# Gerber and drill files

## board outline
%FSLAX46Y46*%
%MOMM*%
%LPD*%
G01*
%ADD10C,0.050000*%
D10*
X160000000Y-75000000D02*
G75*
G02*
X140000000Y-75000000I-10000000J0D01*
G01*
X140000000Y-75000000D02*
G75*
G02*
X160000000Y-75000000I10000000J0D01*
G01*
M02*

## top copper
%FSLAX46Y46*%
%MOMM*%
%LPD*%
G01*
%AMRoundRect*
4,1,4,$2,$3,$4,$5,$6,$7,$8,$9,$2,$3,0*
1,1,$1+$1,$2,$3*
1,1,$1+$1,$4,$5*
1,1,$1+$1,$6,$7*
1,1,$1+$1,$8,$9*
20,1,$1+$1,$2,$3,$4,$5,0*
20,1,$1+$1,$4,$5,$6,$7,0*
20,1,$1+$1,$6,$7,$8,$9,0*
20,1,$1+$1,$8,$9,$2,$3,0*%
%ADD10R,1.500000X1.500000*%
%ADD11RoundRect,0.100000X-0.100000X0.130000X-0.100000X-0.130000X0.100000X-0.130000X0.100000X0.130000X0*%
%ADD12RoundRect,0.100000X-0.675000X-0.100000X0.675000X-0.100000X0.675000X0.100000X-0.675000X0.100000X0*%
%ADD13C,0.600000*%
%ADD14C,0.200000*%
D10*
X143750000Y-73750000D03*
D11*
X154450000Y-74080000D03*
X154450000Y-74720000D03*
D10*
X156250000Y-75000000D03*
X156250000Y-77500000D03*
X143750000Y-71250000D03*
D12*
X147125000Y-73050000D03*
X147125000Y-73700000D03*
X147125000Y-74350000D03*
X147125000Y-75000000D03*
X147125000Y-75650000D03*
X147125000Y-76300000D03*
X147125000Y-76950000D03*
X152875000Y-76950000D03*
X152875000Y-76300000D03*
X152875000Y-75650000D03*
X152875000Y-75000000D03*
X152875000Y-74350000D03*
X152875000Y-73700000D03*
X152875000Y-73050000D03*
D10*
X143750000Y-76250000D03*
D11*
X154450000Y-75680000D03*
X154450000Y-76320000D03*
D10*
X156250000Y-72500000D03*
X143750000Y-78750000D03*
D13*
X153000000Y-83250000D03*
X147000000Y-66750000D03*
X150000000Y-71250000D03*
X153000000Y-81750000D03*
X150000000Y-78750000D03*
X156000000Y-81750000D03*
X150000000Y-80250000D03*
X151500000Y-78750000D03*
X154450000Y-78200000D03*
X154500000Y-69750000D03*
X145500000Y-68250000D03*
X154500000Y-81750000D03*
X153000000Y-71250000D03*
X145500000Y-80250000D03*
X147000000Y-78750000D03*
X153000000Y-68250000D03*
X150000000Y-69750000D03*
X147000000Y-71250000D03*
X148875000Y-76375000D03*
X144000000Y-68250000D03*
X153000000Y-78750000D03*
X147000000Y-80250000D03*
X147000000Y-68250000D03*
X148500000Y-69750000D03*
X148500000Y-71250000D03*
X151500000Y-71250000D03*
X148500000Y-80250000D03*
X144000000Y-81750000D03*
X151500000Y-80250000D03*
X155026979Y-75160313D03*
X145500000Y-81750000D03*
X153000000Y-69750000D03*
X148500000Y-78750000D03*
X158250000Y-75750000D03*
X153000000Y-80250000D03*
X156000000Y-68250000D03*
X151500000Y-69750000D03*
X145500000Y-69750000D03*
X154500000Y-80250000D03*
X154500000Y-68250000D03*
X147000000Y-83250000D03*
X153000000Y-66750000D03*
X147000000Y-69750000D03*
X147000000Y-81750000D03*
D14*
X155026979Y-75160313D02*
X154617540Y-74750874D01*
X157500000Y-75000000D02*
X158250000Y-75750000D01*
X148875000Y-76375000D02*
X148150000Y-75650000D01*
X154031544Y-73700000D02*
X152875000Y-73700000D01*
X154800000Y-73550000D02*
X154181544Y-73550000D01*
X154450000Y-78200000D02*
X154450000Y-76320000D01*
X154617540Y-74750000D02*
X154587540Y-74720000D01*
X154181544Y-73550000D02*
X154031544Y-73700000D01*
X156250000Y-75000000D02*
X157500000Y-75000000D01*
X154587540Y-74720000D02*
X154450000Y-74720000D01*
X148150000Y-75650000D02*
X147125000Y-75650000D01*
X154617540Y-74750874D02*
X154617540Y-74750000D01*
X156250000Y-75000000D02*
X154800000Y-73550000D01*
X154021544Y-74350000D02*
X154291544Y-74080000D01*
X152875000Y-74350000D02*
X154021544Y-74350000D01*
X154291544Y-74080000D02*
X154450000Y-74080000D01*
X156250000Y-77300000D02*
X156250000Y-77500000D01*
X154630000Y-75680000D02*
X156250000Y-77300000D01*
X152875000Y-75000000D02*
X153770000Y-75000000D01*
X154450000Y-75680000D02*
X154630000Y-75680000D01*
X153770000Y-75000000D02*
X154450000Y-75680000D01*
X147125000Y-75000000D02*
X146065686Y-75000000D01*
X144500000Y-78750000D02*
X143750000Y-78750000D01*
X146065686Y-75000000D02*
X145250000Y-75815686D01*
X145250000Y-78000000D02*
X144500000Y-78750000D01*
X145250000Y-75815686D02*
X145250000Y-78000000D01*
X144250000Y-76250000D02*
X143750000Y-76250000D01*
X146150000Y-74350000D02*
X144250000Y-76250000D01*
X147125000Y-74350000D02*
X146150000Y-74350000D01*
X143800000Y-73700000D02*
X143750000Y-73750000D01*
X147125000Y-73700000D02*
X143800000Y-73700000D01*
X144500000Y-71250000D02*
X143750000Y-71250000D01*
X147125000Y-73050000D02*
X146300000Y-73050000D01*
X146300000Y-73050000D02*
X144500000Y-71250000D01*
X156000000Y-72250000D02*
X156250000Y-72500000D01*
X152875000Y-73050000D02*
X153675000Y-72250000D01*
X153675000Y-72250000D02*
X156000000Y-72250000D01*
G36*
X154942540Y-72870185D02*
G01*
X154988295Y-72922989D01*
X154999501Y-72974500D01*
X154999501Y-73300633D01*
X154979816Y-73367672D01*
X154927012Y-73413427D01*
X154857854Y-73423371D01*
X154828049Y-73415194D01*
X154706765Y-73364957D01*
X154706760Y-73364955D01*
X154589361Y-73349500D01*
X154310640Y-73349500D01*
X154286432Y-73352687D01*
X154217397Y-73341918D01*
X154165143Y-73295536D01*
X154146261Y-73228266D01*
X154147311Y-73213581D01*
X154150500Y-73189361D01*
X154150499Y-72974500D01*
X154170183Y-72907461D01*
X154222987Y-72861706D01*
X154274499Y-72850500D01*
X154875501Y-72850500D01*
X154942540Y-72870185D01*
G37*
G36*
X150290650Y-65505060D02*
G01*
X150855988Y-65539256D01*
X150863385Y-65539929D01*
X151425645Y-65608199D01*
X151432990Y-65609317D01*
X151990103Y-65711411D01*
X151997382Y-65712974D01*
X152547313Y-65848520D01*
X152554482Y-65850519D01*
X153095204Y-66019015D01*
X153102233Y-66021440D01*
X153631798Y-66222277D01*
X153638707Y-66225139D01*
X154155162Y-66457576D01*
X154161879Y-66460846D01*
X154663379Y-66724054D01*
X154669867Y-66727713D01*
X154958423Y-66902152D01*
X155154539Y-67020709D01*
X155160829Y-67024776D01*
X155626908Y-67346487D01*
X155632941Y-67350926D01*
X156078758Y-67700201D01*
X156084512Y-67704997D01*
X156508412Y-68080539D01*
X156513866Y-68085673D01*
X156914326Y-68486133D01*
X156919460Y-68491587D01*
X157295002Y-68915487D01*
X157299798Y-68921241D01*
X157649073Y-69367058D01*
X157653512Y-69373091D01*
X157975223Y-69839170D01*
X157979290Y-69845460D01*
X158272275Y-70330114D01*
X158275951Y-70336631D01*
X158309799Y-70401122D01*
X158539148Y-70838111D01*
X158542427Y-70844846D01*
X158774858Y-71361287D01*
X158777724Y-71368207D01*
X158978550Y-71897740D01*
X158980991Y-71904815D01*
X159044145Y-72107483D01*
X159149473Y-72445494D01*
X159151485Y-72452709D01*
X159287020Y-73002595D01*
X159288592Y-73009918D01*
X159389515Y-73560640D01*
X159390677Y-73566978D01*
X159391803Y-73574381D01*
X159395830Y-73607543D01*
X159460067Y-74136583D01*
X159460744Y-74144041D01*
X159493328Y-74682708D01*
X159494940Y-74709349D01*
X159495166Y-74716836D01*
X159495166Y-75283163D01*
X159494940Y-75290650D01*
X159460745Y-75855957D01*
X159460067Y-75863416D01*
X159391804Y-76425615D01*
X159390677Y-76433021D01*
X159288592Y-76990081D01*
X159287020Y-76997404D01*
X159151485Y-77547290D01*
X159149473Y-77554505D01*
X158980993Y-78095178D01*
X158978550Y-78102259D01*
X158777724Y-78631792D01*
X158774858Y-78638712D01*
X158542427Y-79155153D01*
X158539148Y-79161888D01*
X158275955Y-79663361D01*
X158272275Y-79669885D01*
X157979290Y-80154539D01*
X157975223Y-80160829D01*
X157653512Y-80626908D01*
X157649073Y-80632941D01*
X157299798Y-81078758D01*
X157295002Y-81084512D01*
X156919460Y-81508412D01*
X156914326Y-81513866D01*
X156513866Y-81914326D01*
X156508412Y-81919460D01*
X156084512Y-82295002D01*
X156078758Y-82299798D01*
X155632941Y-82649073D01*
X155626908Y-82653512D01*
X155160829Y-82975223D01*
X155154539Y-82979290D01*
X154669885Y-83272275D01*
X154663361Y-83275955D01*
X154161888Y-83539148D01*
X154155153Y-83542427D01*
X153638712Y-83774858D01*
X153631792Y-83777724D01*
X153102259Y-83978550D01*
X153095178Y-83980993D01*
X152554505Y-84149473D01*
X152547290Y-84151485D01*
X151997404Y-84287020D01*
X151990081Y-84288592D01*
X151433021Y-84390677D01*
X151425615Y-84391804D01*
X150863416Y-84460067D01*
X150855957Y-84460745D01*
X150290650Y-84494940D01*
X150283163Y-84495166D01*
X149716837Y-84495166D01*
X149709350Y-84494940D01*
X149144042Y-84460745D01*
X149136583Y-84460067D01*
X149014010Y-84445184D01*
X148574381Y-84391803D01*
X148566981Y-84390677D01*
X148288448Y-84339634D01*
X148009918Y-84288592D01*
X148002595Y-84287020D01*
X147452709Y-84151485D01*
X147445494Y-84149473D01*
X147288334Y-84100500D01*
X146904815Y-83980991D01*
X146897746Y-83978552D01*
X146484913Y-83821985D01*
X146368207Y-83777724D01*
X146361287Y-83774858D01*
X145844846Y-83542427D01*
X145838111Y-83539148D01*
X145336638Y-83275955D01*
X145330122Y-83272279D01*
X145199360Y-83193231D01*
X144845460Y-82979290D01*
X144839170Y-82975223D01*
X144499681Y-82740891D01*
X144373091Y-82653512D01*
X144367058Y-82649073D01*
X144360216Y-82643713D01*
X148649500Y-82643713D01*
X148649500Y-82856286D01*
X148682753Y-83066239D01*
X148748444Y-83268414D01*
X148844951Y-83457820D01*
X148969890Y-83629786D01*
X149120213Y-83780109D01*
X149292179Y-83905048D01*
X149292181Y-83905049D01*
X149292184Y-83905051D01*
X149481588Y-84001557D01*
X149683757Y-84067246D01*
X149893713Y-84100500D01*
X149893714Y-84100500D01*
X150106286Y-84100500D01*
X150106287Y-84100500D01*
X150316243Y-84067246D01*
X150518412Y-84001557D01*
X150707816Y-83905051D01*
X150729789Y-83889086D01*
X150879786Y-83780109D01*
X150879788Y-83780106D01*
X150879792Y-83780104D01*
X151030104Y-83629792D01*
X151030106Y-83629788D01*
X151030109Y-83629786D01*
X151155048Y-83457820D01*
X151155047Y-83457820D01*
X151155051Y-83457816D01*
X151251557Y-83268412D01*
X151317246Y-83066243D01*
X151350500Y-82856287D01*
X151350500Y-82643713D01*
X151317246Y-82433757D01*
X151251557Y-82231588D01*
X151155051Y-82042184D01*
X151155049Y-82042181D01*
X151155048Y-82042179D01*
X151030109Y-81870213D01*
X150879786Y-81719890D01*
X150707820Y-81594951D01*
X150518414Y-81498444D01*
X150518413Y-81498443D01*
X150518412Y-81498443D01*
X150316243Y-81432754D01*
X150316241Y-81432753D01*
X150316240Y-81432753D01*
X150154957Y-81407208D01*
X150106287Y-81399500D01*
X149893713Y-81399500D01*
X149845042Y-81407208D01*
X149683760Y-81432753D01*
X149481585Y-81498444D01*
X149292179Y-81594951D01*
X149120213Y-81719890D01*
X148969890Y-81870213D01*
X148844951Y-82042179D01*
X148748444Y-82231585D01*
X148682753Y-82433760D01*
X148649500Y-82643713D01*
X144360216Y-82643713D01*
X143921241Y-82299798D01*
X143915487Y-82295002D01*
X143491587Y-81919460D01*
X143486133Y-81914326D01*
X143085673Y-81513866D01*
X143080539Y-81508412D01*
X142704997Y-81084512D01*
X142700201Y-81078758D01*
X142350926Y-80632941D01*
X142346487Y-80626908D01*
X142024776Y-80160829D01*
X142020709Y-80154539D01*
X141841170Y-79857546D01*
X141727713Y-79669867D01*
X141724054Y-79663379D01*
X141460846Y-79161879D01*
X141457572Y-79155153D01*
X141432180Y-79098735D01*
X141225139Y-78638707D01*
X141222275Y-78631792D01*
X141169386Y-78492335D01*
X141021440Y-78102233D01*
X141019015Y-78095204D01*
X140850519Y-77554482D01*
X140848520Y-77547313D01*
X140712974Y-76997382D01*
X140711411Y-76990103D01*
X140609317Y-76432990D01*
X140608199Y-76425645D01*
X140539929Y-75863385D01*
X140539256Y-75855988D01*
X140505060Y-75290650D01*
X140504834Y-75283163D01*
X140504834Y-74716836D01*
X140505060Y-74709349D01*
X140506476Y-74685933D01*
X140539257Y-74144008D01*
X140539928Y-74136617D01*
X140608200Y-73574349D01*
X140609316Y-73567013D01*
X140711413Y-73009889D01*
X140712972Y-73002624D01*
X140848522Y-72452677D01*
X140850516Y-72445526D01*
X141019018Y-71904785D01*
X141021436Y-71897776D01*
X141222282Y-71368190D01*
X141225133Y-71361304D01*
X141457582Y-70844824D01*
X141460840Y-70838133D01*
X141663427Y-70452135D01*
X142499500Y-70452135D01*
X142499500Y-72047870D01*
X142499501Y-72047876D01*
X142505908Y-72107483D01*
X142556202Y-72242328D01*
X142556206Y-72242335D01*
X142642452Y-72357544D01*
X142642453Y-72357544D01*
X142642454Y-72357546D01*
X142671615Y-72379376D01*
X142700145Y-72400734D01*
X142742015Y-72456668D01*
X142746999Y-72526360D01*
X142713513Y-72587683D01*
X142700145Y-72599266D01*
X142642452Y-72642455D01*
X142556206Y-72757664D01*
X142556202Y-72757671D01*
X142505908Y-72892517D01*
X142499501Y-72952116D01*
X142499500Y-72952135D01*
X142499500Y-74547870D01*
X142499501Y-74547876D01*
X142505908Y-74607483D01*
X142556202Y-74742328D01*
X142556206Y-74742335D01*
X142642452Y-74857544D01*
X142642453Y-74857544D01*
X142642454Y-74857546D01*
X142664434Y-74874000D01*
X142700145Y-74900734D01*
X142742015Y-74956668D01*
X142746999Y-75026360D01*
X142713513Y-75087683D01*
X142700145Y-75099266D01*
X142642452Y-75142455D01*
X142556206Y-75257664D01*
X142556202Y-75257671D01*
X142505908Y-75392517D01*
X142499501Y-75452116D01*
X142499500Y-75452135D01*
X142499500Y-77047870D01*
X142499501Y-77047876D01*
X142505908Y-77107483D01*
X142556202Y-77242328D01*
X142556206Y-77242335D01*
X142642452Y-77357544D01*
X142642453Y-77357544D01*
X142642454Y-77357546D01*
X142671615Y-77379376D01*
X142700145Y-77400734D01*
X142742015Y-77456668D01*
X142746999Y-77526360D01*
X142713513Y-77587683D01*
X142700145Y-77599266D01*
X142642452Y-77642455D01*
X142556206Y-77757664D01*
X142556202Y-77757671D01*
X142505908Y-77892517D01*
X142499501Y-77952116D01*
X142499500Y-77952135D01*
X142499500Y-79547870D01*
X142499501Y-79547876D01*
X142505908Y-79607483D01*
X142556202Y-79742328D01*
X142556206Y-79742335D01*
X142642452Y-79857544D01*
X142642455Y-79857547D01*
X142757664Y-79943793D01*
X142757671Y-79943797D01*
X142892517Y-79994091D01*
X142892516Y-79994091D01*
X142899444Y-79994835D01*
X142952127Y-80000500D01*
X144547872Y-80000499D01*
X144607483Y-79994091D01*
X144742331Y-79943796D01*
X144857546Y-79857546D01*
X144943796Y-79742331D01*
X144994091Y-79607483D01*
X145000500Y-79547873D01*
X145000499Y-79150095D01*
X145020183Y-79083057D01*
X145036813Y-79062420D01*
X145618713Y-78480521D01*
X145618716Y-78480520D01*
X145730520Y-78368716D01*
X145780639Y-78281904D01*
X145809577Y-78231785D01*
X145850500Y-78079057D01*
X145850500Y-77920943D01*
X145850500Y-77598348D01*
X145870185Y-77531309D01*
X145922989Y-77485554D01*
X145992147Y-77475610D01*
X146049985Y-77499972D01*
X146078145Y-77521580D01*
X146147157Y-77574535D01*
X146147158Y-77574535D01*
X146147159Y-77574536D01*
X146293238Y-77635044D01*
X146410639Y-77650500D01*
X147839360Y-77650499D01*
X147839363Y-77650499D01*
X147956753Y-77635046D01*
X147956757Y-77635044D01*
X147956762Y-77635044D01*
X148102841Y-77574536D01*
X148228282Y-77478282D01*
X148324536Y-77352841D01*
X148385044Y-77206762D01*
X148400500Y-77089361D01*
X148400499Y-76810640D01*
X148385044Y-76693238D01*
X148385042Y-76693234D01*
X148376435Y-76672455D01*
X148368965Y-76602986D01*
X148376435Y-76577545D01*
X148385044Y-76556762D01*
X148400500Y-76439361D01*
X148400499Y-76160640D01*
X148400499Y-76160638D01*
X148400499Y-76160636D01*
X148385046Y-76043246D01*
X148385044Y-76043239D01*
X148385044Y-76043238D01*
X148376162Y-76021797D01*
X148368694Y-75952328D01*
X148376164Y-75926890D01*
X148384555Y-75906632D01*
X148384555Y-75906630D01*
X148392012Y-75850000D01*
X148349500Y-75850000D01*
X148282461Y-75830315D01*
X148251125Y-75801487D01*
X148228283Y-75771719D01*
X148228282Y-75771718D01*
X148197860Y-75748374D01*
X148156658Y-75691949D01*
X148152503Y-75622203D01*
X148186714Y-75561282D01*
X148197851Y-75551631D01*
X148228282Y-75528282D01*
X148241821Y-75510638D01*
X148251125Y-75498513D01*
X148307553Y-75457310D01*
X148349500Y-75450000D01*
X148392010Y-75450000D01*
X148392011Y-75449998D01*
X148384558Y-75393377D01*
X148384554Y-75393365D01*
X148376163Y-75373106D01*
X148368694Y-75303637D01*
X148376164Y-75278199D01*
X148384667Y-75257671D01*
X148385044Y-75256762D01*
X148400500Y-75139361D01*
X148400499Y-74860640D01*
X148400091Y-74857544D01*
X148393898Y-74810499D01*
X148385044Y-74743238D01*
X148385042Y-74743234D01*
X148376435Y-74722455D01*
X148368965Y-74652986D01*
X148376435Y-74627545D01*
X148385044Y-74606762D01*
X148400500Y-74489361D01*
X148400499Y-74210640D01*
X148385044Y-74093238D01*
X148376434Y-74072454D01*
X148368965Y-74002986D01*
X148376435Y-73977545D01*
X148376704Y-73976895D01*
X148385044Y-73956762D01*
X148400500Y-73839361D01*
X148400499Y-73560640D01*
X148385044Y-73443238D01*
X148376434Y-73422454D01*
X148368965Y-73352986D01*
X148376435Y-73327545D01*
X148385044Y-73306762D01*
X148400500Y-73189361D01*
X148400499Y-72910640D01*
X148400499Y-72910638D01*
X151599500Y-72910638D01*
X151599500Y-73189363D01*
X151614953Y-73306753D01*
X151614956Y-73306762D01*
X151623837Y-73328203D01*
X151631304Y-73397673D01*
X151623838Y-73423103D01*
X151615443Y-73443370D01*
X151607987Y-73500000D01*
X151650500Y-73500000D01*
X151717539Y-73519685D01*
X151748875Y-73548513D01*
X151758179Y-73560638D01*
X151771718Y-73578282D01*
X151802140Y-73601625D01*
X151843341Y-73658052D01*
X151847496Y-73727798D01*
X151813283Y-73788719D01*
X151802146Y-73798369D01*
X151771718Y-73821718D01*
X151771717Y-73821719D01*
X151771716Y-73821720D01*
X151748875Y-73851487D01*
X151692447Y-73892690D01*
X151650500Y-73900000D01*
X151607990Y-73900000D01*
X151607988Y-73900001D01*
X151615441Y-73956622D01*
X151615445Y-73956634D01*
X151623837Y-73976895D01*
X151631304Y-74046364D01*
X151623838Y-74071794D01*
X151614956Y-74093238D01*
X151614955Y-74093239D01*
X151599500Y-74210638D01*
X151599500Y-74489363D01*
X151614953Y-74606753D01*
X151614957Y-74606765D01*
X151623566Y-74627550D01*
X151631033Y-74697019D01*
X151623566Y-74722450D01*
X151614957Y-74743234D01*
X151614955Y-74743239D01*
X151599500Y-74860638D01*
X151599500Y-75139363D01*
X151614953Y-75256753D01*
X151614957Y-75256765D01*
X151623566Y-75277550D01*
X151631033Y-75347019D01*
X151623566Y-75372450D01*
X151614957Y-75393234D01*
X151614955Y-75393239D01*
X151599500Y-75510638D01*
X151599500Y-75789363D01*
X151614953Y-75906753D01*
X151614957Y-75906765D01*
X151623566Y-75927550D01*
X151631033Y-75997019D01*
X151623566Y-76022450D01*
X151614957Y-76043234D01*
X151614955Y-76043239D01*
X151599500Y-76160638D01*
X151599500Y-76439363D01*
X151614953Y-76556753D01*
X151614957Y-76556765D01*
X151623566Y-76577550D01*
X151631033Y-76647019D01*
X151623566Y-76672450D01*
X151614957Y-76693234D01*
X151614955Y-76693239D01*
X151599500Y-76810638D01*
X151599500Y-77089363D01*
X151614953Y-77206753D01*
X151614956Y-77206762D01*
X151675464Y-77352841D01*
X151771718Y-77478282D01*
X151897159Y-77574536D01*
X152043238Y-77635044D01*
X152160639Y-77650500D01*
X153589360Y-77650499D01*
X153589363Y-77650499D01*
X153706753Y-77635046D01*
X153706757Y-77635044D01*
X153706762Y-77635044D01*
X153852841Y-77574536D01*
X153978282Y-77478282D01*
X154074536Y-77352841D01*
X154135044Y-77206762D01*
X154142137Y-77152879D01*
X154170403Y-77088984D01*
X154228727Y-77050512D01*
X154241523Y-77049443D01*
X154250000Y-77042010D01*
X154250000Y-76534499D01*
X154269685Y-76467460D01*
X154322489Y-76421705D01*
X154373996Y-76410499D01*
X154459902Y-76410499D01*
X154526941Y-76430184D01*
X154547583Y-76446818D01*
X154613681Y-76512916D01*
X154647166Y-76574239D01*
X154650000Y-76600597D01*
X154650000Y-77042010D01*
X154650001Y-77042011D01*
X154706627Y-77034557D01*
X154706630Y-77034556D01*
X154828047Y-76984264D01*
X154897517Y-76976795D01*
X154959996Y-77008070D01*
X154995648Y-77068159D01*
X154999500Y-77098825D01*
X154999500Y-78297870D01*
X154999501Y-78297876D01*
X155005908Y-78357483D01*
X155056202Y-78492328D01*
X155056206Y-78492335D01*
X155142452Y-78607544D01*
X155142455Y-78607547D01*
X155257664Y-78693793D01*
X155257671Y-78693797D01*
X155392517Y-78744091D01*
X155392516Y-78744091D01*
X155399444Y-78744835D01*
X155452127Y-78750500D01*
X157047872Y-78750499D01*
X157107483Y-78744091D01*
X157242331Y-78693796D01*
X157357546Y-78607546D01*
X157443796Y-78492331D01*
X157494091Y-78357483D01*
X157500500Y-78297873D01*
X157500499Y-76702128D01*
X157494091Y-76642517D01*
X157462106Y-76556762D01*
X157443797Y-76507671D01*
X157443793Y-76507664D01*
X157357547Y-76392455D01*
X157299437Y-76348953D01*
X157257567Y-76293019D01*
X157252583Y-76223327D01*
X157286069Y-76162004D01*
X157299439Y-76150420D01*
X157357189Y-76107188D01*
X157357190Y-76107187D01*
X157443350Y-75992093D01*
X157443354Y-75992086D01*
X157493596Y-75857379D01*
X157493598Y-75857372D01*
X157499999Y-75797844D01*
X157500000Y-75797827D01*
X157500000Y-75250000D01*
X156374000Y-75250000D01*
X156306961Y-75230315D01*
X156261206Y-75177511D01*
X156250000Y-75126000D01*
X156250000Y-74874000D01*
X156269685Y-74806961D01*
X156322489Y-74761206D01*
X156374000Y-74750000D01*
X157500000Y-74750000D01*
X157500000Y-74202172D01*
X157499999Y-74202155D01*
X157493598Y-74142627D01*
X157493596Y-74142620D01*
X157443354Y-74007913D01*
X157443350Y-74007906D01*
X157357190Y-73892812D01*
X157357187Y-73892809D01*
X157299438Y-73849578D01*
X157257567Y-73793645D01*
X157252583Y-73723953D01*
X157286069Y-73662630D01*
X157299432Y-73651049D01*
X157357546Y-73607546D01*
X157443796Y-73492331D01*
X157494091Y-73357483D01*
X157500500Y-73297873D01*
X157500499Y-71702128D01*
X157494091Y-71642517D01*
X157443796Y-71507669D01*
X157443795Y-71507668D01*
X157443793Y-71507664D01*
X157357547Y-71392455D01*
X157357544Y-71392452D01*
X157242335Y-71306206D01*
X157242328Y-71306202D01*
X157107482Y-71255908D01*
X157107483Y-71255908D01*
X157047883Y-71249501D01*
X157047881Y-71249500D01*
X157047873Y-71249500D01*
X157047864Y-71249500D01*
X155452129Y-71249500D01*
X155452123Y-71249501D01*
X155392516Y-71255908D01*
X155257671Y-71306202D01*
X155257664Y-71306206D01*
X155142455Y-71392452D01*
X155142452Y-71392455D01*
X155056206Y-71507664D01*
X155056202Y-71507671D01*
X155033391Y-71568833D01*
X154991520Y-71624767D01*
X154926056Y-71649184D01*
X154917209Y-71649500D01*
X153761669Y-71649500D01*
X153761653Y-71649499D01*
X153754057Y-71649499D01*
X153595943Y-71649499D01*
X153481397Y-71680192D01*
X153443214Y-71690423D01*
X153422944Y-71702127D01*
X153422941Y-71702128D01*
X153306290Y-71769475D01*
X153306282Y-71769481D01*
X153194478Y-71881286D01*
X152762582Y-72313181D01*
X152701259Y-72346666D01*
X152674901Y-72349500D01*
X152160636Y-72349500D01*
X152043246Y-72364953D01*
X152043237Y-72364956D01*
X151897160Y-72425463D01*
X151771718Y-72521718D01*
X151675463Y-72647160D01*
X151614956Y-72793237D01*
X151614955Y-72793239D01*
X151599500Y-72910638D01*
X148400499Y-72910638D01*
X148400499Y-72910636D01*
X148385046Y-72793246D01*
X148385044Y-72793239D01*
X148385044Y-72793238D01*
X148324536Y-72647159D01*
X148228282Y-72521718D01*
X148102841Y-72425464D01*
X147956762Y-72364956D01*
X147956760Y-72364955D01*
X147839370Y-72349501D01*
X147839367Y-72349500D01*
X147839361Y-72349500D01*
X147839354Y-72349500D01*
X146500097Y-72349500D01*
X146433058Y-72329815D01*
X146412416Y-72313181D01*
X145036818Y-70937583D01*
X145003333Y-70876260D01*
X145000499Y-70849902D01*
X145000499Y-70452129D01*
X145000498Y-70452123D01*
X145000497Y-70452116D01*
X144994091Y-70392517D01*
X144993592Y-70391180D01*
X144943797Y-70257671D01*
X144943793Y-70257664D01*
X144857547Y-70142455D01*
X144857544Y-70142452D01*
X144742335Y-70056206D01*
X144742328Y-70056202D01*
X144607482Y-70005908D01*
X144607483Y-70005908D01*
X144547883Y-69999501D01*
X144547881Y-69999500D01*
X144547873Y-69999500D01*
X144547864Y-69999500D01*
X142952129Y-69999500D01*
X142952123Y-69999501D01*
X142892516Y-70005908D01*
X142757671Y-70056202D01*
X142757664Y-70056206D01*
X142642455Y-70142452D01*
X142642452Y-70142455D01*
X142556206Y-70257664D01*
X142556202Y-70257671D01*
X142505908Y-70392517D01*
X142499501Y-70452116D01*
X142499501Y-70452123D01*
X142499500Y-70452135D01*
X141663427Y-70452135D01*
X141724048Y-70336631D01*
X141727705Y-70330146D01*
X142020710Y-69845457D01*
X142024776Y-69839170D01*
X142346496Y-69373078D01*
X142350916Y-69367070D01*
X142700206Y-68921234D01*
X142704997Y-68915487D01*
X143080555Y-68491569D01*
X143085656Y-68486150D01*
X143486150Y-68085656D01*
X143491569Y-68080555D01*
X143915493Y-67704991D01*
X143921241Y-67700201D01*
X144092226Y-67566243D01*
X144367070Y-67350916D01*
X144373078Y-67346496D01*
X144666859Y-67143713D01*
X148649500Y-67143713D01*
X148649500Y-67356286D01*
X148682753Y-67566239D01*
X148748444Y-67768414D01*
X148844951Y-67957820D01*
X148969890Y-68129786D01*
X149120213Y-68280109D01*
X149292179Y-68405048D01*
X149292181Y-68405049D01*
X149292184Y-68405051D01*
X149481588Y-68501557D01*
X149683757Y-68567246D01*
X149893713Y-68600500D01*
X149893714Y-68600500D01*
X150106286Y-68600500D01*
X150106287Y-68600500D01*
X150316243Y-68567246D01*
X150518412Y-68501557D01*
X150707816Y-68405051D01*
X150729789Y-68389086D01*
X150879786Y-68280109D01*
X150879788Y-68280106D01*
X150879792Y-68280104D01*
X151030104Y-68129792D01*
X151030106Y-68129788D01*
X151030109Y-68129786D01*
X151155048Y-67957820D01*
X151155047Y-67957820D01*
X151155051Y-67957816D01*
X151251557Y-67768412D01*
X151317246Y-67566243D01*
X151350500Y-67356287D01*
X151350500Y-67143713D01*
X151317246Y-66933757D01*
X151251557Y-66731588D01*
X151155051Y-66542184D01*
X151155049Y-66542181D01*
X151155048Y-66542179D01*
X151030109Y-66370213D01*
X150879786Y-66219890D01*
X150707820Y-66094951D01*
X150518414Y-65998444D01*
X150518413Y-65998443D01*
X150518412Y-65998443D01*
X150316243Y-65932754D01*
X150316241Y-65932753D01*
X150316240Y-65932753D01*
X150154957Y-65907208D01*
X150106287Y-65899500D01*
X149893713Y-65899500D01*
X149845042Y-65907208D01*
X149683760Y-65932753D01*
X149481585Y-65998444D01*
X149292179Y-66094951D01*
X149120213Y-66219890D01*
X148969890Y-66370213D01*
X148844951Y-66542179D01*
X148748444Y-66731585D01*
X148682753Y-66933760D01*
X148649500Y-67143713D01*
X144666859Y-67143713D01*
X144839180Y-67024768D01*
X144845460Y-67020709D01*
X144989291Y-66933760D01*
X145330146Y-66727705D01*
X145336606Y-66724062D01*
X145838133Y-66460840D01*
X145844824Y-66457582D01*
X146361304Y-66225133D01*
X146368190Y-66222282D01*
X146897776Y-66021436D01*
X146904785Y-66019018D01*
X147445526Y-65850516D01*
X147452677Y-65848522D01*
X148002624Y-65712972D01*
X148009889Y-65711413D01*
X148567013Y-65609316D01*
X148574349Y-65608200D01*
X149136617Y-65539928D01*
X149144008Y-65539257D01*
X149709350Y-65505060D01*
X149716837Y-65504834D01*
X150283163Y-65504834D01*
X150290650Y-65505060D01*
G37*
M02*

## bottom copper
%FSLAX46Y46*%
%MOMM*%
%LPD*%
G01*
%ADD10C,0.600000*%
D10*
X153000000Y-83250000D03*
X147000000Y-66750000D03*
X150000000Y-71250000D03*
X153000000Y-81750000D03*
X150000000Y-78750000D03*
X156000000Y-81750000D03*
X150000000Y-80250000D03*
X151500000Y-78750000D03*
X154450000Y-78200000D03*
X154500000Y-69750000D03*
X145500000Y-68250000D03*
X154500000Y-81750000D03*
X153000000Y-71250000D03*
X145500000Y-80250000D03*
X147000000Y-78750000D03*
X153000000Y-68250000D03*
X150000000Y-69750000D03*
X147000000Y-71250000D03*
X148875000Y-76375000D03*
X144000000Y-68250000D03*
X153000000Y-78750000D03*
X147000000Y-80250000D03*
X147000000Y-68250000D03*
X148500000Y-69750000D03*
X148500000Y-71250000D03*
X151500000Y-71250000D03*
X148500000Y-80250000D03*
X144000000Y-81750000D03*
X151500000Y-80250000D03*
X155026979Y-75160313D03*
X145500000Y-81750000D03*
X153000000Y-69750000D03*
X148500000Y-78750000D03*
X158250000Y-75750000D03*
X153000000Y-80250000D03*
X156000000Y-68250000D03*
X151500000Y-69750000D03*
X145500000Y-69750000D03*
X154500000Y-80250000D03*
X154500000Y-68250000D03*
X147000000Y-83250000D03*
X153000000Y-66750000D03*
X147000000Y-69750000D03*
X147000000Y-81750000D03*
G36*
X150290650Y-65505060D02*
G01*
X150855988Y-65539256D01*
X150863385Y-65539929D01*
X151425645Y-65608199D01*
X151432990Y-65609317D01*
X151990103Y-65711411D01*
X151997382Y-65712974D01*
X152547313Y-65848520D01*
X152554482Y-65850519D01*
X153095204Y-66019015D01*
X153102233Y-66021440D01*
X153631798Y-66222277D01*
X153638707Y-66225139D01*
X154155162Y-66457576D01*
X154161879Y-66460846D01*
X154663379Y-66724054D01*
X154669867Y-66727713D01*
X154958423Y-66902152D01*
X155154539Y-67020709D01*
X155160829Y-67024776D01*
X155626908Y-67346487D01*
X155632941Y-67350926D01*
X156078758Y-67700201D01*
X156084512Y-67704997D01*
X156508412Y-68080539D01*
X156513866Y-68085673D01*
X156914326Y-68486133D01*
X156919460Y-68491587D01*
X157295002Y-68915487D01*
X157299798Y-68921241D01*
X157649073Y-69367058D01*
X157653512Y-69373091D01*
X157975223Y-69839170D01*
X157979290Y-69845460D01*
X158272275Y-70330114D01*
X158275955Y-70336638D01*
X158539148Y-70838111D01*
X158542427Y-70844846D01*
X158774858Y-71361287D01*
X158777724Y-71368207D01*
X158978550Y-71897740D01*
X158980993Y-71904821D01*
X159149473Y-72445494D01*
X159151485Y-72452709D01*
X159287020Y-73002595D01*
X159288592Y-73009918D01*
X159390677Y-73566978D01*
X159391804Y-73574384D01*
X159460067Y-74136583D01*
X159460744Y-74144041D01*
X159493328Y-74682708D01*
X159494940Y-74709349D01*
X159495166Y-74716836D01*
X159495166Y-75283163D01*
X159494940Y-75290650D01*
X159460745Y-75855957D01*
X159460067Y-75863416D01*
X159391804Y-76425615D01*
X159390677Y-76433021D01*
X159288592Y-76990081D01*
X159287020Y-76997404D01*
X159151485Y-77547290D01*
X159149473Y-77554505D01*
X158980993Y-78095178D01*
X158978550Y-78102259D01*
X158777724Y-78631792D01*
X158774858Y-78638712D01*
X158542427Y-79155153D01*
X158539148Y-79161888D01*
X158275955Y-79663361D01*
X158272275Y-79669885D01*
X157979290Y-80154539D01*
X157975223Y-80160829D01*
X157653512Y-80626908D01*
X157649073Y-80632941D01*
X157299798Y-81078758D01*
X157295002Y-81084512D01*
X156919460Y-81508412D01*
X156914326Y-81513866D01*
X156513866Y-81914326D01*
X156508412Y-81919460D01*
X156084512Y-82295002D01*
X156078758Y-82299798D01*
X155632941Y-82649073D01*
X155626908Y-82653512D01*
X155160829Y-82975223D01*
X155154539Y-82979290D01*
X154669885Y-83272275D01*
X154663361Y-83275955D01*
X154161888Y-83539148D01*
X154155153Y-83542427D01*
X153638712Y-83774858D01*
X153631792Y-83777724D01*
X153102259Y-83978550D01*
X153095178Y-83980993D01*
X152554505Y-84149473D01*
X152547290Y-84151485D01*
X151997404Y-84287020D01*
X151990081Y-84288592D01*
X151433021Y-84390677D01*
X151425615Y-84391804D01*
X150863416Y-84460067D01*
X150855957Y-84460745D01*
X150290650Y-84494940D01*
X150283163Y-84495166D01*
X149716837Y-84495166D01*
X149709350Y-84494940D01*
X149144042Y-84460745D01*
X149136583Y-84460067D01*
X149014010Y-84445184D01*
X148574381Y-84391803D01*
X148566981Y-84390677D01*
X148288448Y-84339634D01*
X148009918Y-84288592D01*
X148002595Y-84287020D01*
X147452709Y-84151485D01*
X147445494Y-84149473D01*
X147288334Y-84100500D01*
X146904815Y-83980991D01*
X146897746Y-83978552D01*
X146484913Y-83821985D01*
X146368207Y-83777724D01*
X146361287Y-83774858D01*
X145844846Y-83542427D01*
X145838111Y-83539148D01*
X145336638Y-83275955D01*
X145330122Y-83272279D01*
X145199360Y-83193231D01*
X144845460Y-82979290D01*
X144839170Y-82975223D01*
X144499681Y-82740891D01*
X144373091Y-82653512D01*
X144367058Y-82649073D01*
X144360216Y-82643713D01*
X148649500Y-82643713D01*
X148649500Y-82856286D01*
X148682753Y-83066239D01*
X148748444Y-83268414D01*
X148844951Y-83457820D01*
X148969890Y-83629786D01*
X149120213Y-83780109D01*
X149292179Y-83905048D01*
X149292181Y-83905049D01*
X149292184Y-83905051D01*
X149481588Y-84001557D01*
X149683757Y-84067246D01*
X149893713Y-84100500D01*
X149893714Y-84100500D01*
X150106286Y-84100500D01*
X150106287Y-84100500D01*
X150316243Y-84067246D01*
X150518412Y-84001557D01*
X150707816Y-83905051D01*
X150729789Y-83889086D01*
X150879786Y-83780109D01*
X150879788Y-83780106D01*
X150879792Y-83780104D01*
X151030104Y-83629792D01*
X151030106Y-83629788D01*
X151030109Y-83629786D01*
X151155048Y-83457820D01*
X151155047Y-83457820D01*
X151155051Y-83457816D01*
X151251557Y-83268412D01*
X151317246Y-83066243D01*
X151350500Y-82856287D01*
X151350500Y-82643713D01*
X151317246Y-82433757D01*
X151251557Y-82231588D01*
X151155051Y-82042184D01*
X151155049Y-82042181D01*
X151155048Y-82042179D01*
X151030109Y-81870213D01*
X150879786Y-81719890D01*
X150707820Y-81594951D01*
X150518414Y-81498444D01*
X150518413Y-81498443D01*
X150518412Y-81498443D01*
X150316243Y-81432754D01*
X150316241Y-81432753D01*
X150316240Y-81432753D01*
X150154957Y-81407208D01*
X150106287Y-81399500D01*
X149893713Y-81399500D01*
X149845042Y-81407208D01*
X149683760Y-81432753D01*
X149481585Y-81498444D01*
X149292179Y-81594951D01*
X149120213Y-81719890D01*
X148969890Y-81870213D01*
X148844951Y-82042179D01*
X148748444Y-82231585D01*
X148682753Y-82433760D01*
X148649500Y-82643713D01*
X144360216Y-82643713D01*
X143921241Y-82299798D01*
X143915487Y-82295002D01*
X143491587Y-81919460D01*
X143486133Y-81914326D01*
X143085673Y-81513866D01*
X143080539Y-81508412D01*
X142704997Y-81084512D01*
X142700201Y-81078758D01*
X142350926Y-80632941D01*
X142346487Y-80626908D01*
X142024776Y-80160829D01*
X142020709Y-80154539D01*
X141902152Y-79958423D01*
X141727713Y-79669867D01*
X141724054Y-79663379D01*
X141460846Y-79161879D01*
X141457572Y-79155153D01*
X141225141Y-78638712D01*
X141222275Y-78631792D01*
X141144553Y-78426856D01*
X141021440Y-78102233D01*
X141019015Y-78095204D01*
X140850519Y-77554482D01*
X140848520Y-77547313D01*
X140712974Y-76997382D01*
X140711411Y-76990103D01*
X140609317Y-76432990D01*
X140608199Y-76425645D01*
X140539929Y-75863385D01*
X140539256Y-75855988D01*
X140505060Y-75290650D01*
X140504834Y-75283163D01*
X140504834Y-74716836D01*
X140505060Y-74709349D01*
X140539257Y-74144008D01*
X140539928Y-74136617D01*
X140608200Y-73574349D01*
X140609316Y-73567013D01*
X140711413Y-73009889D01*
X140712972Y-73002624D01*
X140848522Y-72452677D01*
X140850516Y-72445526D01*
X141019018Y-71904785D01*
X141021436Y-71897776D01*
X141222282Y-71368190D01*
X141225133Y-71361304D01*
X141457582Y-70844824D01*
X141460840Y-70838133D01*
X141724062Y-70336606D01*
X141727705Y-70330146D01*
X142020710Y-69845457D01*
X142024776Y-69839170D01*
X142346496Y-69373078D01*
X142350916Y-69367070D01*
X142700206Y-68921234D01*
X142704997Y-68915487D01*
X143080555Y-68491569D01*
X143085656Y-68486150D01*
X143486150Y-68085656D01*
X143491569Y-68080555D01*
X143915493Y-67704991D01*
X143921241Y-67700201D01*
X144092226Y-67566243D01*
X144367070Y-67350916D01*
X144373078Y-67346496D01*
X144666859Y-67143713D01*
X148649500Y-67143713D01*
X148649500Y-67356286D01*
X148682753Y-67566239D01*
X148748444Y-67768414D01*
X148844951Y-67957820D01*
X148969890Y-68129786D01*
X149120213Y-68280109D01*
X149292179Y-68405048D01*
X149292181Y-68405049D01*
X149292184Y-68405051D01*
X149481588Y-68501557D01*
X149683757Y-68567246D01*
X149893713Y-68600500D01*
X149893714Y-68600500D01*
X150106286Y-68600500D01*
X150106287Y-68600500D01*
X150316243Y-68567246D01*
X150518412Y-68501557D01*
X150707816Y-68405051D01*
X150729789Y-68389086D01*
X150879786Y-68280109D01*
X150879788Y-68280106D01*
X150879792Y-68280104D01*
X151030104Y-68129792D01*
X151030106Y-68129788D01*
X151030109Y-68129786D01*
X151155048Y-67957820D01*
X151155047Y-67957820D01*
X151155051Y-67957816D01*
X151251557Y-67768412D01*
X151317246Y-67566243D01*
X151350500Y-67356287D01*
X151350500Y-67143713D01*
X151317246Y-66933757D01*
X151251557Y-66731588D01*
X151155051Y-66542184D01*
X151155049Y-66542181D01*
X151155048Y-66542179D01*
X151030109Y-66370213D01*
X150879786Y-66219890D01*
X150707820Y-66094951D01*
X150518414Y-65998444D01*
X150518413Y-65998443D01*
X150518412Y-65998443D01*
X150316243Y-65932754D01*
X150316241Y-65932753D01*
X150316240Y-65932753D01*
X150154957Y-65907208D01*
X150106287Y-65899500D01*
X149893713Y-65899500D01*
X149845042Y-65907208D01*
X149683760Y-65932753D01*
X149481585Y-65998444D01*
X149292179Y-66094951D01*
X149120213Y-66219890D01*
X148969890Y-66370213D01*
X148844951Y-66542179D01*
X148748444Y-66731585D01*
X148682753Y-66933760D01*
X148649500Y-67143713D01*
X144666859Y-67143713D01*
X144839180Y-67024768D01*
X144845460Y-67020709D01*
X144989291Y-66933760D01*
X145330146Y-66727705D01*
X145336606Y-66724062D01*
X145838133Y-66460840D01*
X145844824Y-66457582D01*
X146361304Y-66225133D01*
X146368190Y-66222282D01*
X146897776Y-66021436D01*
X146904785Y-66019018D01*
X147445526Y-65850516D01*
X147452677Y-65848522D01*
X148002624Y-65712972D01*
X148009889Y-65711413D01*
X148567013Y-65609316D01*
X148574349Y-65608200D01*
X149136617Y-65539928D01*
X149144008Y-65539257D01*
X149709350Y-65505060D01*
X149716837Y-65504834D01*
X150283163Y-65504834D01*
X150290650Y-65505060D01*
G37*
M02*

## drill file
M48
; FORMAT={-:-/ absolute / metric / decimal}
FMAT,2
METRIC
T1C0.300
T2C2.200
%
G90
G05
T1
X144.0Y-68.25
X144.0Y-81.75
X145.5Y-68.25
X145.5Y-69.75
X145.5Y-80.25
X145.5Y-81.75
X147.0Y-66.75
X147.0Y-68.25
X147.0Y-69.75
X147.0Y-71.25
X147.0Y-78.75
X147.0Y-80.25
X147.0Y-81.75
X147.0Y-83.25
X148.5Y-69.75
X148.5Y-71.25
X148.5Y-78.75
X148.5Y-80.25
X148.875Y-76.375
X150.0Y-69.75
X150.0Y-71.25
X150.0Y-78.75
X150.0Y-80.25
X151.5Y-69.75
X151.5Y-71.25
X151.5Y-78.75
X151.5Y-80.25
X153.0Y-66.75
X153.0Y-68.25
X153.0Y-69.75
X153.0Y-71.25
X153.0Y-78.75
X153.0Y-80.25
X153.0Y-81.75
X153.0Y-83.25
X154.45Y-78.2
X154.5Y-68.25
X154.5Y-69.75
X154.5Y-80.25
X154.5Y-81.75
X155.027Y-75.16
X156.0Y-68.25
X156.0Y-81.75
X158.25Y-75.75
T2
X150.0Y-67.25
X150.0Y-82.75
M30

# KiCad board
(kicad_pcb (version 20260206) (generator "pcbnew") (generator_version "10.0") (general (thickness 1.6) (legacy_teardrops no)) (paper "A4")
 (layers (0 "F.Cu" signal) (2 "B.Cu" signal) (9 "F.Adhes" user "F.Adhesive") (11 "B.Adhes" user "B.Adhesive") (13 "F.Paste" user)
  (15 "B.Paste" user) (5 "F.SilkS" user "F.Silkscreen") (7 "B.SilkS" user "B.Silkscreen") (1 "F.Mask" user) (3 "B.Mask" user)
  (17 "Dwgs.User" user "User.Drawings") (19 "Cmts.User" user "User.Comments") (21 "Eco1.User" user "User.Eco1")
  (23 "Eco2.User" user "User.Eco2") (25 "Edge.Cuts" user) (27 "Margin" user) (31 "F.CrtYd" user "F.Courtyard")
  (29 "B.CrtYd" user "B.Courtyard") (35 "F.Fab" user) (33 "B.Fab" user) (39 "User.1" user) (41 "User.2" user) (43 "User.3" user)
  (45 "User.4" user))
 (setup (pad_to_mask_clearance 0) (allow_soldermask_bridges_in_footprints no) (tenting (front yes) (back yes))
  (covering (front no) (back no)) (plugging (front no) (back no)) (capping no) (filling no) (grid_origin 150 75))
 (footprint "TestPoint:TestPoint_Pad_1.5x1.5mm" (layer "F.Cu") (at 143.75 73.75 180)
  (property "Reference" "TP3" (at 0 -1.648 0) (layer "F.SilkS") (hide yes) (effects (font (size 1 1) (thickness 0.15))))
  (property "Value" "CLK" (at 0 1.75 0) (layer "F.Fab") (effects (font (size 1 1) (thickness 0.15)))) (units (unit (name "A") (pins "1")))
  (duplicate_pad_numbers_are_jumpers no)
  (pad "1" smd rect (at 0 0 180) (size 1.5 1.5) (layers "F.Cu" "F.Mask") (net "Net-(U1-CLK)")))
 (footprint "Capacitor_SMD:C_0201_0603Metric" (layer "F.Cu") (at 154.45 74.4 -90)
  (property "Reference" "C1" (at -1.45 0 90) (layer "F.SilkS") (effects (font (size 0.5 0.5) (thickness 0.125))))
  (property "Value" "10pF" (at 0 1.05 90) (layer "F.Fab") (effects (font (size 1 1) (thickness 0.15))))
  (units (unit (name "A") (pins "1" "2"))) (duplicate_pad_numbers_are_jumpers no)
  (pad "" smd roundrect (at -0.345 0 270) (size 0.318 0.36) (layers "F.Paste") (roundrect_rratio 0.25))
  (pad "" smd roundrect (at 0.345 0 270) (size 0.318 0.36) (layers "F.Paste") (roundrect_rratio 0.25))
  (pad "1" smd roundrect (at -0.32 0 270) (size 0.46 0.4) (layers "F.Cu" "F.Mask") (roundrect_rratio 0.25) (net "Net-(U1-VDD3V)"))
  (pad "2" smd roundrect (at 0.32 0 270) (size 0.46 0.4) (layers "F.Cu" "F.Mask") (roundrect_rratio 0.25) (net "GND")))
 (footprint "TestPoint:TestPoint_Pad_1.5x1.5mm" (layer "F.Cu") (at 156.25 75)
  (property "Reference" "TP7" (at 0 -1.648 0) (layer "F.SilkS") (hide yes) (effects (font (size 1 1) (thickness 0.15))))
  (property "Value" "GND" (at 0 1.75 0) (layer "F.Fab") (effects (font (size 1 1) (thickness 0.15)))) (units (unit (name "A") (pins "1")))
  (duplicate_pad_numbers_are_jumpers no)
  (pad "1" smd rect (at 0 0) (size 1.5 1.5) (layers "F.Cu" "F.Mask") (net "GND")))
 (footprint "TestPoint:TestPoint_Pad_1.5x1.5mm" (layer "F.Cu") (at 156.25 77.5)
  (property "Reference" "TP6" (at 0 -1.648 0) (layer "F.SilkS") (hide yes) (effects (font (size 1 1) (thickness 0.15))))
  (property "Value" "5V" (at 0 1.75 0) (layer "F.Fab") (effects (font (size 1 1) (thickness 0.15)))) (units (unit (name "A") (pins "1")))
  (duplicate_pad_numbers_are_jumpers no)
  (pad "1" smd rect (at 0 0) (size 1.5 1.5) (layers "F.Cu" "F.Mask") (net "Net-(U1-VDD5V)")))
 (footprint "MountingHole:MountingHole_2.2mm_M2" (layer "F.Cu") (at 150 82.75)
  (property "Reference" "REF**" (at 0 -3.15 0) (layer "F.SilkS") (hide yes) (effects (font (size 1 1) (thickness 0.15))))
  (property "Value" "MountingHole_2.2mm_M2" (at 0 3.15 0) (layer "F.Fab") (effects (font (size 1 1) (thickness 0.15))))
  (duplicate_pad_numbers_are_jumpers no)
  (pad "" np_thru_hole circle (at 0 0) (size 2.2 2.2) (drill 2.2) (layers "*.Cu" "*.Mask")))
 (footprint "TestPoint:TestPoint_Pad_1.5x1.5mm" (layer "F.Cu") (at 143.75 71.25 180)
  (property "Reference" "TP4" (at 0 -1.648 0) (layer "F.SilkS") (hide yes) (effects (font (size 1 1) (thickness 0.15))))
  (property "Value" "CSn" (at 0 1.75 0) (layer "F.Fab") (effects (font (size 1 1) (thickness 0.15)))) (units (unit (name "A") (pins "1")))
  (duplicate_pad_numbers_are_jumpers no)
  (pad "1" smd rect (at 0 0 180) (size 1.5 1.5) (layers "F.Cu" "F.Mask") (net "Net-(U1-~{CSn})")))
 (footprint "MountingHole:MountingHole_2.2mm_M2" (layer "F.Cu") (at 150 67.25)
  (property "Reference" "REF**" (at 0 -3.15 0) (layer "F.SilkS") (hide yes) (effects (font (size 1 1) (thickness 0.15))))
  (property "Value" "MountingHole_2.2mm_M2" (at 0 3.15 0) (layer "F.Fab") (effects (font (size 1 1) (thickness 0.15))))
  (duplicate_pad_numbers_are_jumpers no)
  (pad "" np_thru_hole circle (at 0 0) (size 2.2 2.2) (drill 2.2) (layers "*.Cu" "*.Mask")))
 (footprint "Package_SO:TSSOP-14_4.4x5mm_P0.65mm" (layer "F.Cu") (at 150 75)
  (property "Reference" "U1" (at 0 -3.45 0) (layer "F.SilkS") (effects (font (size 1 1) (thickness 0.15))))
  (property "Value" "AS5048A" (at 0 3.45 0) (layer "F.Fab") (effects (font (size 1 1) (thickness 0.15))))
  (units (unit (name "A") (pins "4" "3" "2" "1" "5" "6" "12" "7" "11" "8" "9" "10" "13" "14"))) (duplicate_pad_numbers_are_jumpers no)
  (pad "1" smd roundrect (at -2.875 -1.95) (size 1.55 0.4) (layers "F.Cu" "F.Mask" "F.Paste") (roundrect_rratio 0.25)
   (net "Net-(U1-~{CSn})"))
  (pad "2" smd roundrect (at -2.875 -1.3) (size 1.55 0.4) (layers "F.Cu" "F.Mask" "F.Paste") (roundrect_rratio 0.25) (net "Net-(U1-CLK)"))
  (pad "3" smd roundrect (at -2.875 -0.65) (size 1.55 0.4) (layers "F.Cu" "F.Mask" "F.Paste") (roundrect_rratio 0.25) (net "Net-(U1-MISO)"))
  (pad "4" smd roundrect (at -2.875 0) (size 1.55 0.4) (layers "F.Cu" "F.Mask" "F.Paste") (roundrect_rratio 0.25) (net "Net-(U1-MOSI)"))
  (pad "5" smd roundrect (at -2.875 0.65) (size 1.55 0.4) (layers "F.Cu" "F.Mask" "F.Paste") (roundrect_rratio 0.25) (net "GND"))
  (pad "6" smd roundrect (at -2.875 1.3) (size 1.55 0.4) (layers "F.Cu" "F.Mask" "F.Paste") (roundrect_rratio 0.25)
   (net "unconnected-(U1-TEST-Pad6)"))
  (pad "7" smd roundrect (at -2.875 1.95) (size 1.55 0.4) (layers "F.Cu" "F.Mask" "F.Paste") (roundrect_rratio 0.25)
   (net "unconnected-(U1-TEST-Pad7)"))
  (pad "8" smd roundrect (at 2.875 1.95) (size 1.55 0.4) (layers "F.Cu" "F.Mask" "F.Paste") (roundrect_rratio 0.25)
   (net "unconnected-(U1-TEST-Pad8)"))
  (pad "9" smd roundrect (at 2.875 1.3) (size 1.55 0.4) (layers "F.Cu" "F.Mask" "F.Paste") (roundrect_rratio 0.25)
   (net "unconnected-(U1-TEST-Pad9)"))
  (pad "10" smd roundrect (at 2.875 0.65) (size 1.55 0.4) (layers "F.Cu" "F.Mask" "F.Paste") (roundrect_rratio 0.25)
   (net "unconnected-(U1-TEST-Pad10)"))
  (pad "11" smd roundrect (at 2.875 0) (size 1.55 0.4) (layers "F.Cu" "F.Mask" "F.Paste") (roundrect_rratio 0.25) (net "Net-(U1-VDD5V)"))
  (pad "12" smd roundrect (at 2.875 -0.65) (size 1.55 0.4) (layers "F.Cu" "F.Mask" "F.Paste") (roundrect_rratio 0.25) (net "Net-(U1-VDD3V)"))
  (pad "13" smd roundrect (at 2.875 -1.3) (size 1.55 0.4) (layers "F.Cu" "F.Mask" "F.Paste") (roundrect_rratio 0.25) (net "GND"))
  (pad "14" smd roundrect (at 2.875 -1.95) (size 1.55 0.4) (layers "F.Cu" "F.Mask" "F.Paste") (roundrect_rratio 0.25) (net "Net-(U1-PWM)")))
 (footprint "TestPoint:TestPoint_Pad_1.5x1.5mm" (layer "F.Cu") (at 143.75 76.25 180)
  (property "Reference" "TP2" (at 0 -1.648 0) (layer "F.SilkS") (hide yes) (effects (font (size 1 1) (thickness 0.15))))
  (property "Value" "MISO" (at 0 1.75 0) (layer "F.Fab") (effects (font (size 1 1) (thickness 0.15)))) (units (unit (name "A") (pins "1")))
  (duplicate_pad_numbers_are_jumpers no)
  (pad "1" smd rect (at 0 0 180) (size 1.5 1.5) (layers "F.Cu" "F.Mask") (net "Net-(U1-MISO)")))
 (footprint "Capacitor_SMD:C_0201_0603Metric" (layer "F.Cu") (at 154.45 76 -90)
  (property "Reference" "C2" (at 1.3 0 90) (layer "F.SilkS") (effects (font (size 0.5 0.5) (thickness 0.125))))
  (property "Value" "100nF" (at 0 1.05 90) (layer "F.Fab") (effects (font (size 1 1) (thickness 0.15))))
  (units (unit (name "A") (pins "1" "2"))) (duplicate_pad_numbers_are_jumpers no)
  (pad "" smd roundrect (at -0.345 0 270) (size 0.318 0.36) (layers "F.Paste") (roundrect_rratio 0.25))
  (pad "" smd roundrect (at 0.345 0 270) (size 0.318 0.36) (layers "F.Paste") (roundrect_rratio 0.25))
  (pad "1" smd roundrect (at -0.32 0 270) (size 0.46 0.4) (layers "F.Cu" "F.Mask") (roundrect_rratio 0.25) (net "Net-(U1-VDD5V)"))
  (pad "2" smd roundrect (at 0.32 0 270) (size 0.46 0.4) (layers "F.Cu" "F.Mask") (roundrect_rratio 0.25) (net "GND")))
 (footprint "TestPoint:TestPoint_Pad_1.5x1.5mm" (layer "F.Cu") (at 156.25 72.5)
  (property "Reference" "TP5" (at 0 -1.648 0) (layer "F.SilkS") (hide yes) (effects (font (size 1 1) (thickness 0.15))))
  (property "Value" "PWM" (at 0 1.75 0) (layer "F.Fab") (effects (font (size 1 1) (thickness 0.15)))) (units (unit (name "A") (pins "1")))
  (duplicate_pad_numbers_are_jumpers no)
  (pad "1" smd rect (at 0 0) (size 1.5 1.5) (layers "F.Cu" "F.Mask") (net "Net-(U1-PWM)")))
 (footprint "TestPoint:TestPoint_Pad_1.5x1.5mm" (layer "F.Cu") (at 143.75 78.75 180)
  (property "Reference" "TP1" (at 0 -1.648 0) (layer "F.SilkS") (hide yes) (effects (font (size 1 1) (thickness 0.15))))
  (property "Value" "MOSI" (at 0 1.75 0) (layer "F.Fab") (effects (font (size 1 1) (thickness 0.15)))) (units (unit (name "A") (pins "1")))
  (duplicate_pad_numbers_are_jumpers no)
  (pad "1" smd rect (at 0 0 180) (size 1.5 1.5) (layers "F.Cu" "F.Mask") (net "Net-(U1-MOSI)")))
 (gr_circle (center 150 75) (end 160 75) (stroke (width 0.05) (type solid)) (fill no) (layer "Edge.Cuts"))
 (segment (start 155.026979 75.160313) (end 154.61754 74.750874) (width 0.2) (layer "F.Cu") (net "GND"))
 (segment (start 157.5 75) (end 158.25 75.75) (width 0.2) (layer "F.Cu") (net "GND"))
 (segment (start 148.875 76.375) (end 148.15 75.65) (width 0.2) (layer "F.Cu") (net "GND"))
 (segment (start 154.031544 73.7) (end 152.875 73.7) (width 0.2) (layer "F.Cu") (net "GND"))
 (segment (start 154.8 73.55) (end 154.181544 73.55) (width 0.2) (layer "F.Cu") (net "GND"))
 (segment (start 154.45 78.2) (end 154.45 76.32) (width 0.2) (layer "F.Cu") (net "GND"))
 (segment (start 154.61754 74.75) (end 154.58754 74.72) (width 0.2) (layer "F.Cu") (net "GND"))
 (segment (start 154.181544 73.55) (end 154.031544 73.7) (width 0.2) (layer "F.Cu") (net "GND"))
 (segment (start 156.25 75) (end 157.5 75) (width 0.2) (layer "F.Cu") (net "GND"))
 (segment (start 154.58754 74.72) (end 154.45 74.72) (width 0.2) (layer "F.Cu") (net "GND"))
 (segment (start 148.15 75.65) (end 147.125 75.65) (width 0.2) (layer "F.Cu") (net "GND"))
 (segment (start 154.61754 74.750874) (end 154.61754 74.75) (width 0.2) (layer "F.Cu") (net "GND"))
 (segment (start 156.25 75) (end 154.8 73.55) (width 0.2) (layer "F.Cu") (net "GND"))
 (via (at 153 83.25) (size 0.6) (drill 0.3) (layers "F.Cu" "B.Cu") (free yes) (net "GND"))
 (via (at 147 66.75) (size 0.6) (drill 0.3) (layers "F.Cu" "B.Cu") (free yes) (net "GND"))
 (via (at 150 71.25) (size 0.6) (drill 0.3) (layers "F.Cu" "B.Cu") (free yes) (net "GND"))
 (via (at 153 81.75) (size 0.6) (drill 0.3) (layers "F.Cu" "B.Cu") (free yes) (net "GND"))
 (via (at 150 78.75) (size 0.6) (drill 0.3) (layers "F.Cu" "B.Cu") (free yes) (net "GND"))
 (via (at 156 81.75) (size 0.6) (drill 0.3) (layers "F.Cu" "B.Cu") (free yes) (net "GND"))
 (via (at 150 80.25) (size 0.6) (drill 0.3) (layers "F.Cu" "B.Cu") (free yes) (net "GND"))
 (via (at 151.5 78.75) (size 0.6) (drill 0.3) (layers "F.Cu" "B.Cu") (free yes) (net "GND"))
 (via (at 154.45 78.2) (size 0.6) (drill 0.3) (layers "F.Cu" "B.Cu") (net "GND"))
 (via (at 154.5 69.75) (size 0.6) (drill 0.3) (layers "F.Cu" "B.Cu") (free yes) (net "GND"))
 (via (at 145.5 68.25) (size 0.6) (drill 0.3) (layers "F.Cu" "B.Cu") (free yes) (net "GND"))
 (via (at 154.5 81.75) (size 0.6) (drill 0.3) (layers "F.Cu" "B.Cu") (free yes) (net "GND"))
 (via (at 153 71.25) (size 0.6) (drill 0.3) (layers "F.Cu" "B.Cu") (free yes) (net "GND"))
 (via (at 145.5 80.25) (size 0.6) (drill 0.3) (layers "F.Cu" "B.Cu") (free yes) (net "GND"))
 (via (at 147 78.75) (size 0.6) (drill 0.3) (layers "F.Cu" "B.Cu") (free yes) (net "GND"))
 (via (at 153 68.25) (size 0.6) (drill 0.3) (layers "F.Cu" "B.Cu") (free yes) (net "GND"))
 (via (at 150 69.75) (size 0.6) (drill 0.3) (layers "F.Cu" "B.Cu") (free yes) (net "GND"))
 (via (at 147 71.25) (size 0.6) (drill 0.3) (layers "F.Cu" "B.Cu") (free yes) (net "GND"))
 (via (at 148.875 76.375) (size 0.6) (drill 0.3) (layers "F.Cu" "B.Cu") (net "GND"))
 (via (at 144 68.25) (size 0.6) (drill 0.3) (layers "F.Cu" "B.Cu") (free yes) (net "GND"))
 (via (at 153 78.75) (size 0.6) (drill 0.3) (layers "F.Cu" "B.Cu") (free yes) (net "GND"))
 (via (at 147 80.25) (size 0.6) (drill 0.3) (layers "F.Cu" "B.Cu") (free yes) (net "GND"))
 (via (at 147 68.25) (size 0.6) (drill 0.3) (layers "F.Cu" "B.Cu") (free yes) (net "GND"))
 (via (at 148.5 69.75) (size 0.6) (drill 0.3) (layers "F.Cu" "B.Cu") (free yes) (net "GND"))
 (via (at 148.5 71.25) (size 0.6) (drill 0.3) (layers "F.Cu" "B.Cu") (free yes) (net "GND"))
 (via (at 151.5 71.25) (size 0.6) (drill 0.3) (layers "F.Cu" "B.Cu") (free yes) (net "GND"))
 (via (at 148.5 80.25) (size 0.6) (drill 0.3) (layers "F.Cu" "B.Cu") (free yes) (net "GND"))
 (via (at 144 81.75) (size 0.6) (drill 0.3) (layers "F.Cu" "B.Cu") (free yes) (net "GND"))
 (via (at 151.5 80.25) (size 0.6) (drill 0.3) (layers "F.Cu" "B.Cu") (free yes) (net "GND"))
 (via (at 155.026979 75.160313) (size 0.6) (drill 0.3) (layers "F.Cu" "B.Cu") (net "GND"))
 (via (at 145.5 81.75) (size 0.6) (drill 0.3) (layers "F.Cu" "B.Cu") (free yes) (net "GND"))
 (via (at 153 69.75) (size 0.6) (drill 0.3) (layers "F.Cu" "B.Cu") (free yes) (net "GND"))
 (via (at 148.5 78.75) (size 0.6) (drill 0.3) (layers "F.Cu" "B.Cu") (free yes) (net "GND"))
 (via (at 158.25 75.75) (size 0.6) (drill 0.3) (layers "F.Cu" "B.Cu") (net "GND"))
 (via (at 153 80.25) (size 0.6) (drill 0.3) (layers "F.Cu" "B.Cu") (free yes) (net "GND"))
 (via (at 156 68.25) (size 0.6) (drill 0.3) (layers "F.Cu" "B.Cu") (free yes) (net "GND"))
 (via (at 151.5 69.75) (size 0.6) (drill 0.3) (layers "F.Cu" "B.Cu") (free yes) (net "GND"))
 (via (at 145.5 69.75) (size 0.6) (drill 0.3) (layers "F.Cu" "B.Cu") (free yes) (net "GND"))
 (via (at 154.5 80.25) (size 0.6) (drill 0.3) (layers "F.Cu" "B.Cu") (free yes) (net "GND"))
 (via (at 154.5 68.25) (size 0.6) (drill 0.3) (layers "F.Cu" "B.Cu") (free yes) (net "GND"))
 (via (at 147 83.25) (size 0.6) (drill 0.3) (layers "F.Cu" "B.Cu") (free yes) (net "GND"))
 (via (at 153 66.75) (size 0.6) (drill 0.3) (layers "F.Cu" "B.Cu") (free yes) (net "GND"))
 (via (at 147 69.75) (size 0.6) (drill 0.3) (layers "F.Cu" "B.Cu") (free yes) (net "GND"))
 (via (at 147 81.75) (size 0.6) (drill 0.3) (layers "F.Cu" "B.Cu") (free yes) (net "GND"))
 (segment (start 154.021544 74.35) (end 154.291544 74.08) (width 0.2) (layer "F.Cu") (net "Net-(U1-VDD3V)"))
 (segment (start 152.875 74.35) (end 154.021544 74.35) (width 0.2) (layer "F.Cu") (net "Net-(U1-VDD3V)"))
 (segment (start 154.291544 74.08) (end 154.45 74.08) (width 0.2) (layer "F.Cu") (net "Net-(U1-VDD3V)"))
 (segment (start 156.25 77.3) (end 156.25 77.5) (width 0.2) (layer "F.Cu") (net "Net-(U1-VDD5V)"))
 (segment (start 154.63 75.68) (end 156.25 77.3) (width 0.2) (layer "F.Cu") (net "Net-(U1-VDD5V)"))
 (segment (start 152.875 75) (end 153.77 75) (width 0.2) (layer "F.Cu") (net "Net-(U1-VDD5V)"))
 (segment (start 154.45 75.68) (end 154.63 75.68) (width 0.2) (layer "F.Cu") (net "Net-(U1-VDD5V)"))
 (segment (start 153.77 75) (end 154.45 75.68) (width 0.2) (layer "F.Cu") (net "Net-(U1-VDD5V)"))
 (segment (start 147.125 75) (end 146.065686 75) (width 0.2) (layer "F.Cu") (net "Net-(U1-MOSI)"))
 (segment (start 144.5 78.75) (end 143.75 78.75) (width 0.2) (layer "F.Cu") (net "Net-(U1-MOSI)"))
 (segment (start 146.065686 75) (end 145.25 75.815686) (width 0.2) (layer "F.Cu") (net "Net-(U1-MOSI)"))
 (segment (start 145.25 78) (end 144.5 78.75) (width 0.2) (layer "F.Cu") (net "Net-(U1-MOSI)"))
 (segment (start 145.25 75.815686) (end 145.25 78) (width 0.2) (layer "F.Cu") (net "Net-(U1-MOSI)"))
 (segment (start 144.25 76.25) (end 143.75 76.25) (width 0.2) (layer "F.Cu") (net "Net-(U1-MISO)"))
 (segment (start 146.15 74.35) (end 144.25 76.25) (width 0.2) (layer "F.Cu") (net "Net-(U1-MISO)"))
 (segment (start 147.125 74.35) (end 146.15 74.35) (width 0.2) (layer "F.Cu") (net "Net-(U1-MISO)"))
 (segment (start 143.8 73.7) (end 143.75 73.75) (width 0.2) (layer "F.Cu") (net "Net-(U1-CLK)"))
 (segment (start 147.125 73.7) (end 143.8 73.7) (width 0.2) (layer "F.Cu") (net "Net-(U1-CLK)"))
 (segment (start 144.5 71.25) (end 143.75 71.25) (width 0.2) (layer "F.Cu") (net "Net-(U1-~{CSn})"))
 (segment (start 147.125 73.05) (end 146.3 73.05) (width 0.2) (layer "F.Cu") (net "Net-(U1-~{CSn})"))
 (segment (start 146.3 73.05) (end 144.5 71.25) (width 0.2) (layer "F.Cu") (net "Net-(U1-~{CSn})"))
 (segment (start 156 72.25) (end 156.25 72.5) (width 0.2) (layer "F.Cu") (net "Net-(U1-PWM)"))
 (segment (start 152.875 73.05) (end 153.675 72.25) (width 0.2) (layer "F.Cu") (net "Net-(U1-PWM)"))
 (segment (start 153.675 72.25) (end 156 72.25) (width 0.2) (layer "F.Cu") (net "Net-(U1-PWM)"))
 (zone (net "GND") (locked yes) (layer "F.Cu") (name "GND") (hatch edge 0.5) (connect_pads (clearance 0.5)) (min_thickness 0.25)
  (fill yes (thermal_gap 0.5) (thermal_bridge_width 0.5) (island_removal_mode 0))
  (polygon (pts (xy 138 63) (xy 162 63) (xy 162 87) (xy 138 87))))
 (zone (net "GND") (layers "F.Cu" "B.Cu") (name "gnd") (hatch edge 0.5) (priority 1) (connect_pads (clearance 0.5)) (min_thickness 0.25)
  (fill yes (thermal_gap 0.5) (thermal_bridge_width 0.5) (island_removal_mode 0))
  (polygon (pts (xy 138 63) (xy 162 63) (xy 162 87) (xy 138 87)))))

